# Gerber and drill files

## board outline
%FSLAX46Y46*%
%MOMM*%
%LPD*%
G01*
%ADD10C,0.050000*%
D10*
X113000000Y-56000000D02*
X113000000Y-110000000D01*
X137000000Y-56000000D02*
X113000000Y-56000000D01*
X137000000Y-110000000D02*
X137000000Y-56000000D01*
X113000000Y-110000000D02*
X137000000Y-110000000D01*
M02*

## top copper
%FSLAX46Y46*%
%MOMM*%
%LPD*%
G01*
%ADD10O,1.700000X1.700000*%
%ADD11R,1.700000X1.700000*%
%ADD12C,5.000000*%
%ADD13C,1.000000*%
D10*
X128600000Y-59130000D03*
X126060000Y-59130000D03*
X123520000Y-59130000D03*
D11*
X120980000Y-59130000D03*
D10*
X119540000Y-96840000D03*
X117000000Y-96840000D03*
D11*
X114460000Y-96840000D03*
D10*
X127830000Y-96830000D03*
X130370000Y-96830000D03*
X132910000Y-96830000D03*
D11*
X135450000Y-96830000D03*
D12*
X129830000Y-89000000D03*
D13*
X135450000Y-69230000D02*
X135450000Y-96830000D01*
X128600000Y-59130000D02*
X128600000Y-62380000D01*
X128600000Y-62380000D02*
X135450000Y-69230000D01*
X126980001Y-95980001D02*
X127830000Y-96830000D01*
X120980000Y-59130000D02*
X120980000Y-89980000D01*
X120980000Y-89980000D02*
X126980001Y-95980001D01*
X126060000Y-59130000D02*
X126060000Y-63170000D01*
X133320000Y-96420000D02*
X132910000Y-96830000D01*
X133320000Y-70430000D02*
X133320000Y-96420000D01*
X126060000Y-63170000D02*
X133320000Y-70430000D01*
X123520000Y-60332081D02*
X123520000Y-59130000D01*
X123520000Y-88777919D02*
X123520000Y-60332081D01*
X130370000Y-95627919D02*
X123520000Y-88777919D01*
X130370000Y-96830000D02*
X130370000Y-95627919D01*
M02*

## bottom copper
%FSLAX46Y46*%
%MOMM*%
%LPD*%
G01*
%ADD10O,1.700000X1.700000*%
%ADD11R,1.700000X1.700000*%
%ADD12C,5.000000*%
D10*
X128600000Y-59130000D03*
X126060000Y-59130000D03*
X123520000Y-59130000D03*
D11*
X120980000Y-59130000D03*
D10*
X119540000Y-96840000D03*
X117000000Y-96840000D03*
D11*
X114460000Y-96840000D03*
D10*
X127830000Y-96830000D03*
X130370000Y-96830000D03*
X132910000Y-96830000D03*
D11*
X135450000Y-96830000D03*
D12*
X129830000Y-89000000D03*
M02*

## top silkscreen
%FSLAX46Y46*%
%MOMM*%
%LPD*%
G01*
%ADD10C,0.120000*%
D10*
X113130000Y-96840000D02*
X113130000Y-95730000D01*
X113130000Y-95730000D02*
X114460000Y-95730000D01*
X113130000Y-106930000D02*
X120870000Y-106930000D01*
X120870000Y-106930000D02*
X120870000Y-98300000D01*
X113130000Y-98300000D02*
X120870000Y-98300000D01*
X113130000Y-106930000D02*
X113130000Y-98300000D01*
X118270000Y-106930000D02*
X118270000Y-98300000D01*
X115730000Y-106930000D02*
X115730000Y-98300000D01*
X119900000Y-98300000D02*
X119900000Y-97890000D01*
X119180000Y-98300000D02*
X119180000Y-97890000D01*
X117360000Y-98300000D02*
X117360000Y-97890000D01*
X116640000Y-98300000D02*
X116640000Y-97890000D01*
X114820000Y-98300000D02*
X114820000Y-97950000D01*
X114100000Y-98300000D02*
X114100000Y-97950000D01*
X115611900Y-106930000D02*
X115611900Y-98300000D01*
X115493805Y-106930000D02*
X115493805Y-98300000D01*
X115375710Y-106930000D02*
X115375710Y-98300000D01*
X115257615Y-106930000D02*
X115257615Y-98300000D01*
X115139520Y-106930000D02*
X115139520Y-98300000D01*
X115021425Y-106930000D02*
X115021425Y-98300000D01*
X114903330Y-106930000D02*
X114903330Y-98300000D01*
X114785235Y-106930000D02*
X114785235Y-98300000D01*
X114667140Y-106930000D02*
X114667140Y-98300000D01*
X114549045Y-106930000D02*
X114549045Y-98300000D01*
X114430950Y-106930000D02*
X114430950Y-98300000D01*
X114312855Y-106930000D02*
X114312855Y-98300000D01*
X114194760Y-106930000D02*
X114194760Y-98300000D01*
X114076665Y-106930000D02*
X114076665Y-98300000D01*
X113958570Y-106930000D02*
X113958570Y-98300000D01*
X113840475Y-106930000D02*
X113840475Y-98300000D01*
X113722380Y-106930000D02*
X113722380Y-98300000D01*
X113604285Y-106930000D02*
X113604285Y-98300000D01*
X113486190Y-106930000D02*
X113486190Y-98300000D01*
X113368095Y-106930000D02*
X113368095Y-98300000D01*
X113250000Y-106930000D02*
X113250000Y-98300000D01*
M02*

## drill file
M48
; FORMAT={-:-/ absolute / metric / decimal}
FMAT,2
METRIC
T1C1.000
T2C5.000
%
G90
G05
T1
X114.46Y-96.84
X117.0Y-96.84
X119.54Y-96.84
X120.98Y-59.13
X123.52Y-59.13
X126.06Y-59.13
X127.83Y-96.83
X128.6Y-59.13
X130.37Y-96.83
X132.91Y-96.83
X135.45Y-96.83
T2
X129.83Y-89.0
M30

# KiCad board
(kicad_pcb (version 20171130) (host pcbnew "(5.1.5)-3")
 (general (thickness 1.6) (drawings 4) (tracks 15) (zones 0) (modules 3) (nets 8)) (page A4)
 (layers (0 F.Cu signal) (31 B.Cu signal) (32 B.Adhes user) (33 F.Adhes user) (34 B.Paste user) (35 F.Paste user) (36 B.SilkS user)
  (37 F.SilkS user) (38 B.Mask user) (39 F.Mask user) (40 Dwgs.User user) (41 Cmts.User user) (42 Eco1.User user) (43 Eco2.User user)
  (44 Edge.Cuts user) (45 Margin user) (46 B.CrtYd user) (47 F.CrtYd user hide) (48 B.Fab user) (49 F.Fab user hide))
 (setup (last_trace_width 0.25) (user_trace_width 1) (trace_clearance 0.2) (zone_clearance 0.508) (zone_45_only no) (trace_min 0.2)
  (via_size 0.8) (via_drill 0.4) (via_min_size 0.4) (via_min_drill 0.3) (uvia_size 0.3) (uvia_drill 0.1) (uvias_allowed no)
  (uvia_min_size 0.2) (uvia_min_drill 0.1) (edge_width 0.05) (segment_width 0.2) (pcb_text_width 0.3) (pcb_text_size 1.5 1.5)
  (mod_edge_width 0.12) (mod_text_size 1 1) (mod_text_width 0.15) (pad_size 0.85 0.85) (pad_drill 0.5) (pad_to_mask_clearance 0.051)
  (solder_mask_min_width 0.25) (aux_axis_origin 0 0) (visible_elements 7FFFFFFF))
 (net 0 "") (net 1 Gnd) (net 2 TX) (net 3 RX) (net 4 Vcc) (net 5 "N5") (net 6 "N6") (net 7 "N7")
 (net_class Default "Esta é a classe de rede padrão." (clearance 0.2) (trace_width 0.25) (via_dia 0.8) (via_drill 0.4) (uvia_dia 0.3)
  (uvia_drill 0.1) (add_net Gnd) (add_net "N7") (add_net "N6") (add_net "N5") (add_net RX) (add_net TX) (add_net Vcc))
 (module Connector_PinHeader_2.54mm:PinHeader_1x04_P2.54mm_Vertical (layer B.Cu) (at 120.98 59.13 270)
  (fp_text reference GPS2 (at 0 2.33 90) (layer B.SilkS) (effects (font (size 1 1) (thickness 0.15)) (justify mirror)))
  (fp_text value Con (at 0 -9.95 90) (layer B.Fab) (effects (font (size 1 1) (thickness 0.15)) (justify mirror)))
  (pad 4 thru_hole oval (at 0 -7.62 270) (size 1.7 1.7) (drill 1) (layers *.Cu *.Mask) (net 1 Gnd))
  (pad 3 thru_hole oval (at 0 -5.08 270) (size 1.7 1.7) (drill 1) (layers *.Cu *.Mask) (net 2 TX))
  (pad 2 thru_hole oval (at 0 -2.54 270) (size 1.7 1.7) (drill 1) (layers *.Cu *.Mask) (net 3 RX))
  (pad 1 thru_hole rect (at 0 0 270) (size 1.7 1.7) (drill 1) (layers *.Cu *.Mask) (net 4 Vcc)))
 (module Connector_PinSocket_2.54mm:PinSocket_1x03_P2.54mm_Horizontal (layer F.Cu) (at 114.46 96.84 90)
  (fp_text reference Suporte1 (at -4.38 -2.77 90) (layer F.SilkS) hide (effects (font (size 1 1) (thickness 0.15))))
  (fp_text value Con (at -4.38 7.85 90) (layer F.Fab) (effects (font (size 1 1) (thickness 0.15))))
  (fp_line (start 0 -1.33) (end 1.11 -1.33) (layer F.SilkS) (width 0.12))
  (fp_line (start 1.11 -1.33) (end 1.11 0) (layer F.SilkS) (width 0.12))
  (fp_line (start -10.09 -1.33) (end -10.09 6.41) (layer F.SilkS) (width 0.12))
  (fp_line (start -10.09 6.41) (end -1.46 6.41) (layer F.SilkS) (width 0.12))
  (fp_line (start -1.46 -1.33) (end -1.46 6.41) (layer F.SilkS) (width 0.12))
  (fp_line (start -10.09 -1.33) (end -1.46 -1.33) (layer F.SilkS) (width 0.12))
  (fp_line (start -10.09 3.81) (end -1.46 3.81) (layer F.SilkS) (width 0.12))
  (fp_line (start -10.09 1.27) (end -1.46 1.27) (layer F.SilkS) (width 0.12))
  (fp_line (start -1.46 5.44) (end -1.05 5.44) (layer F.SilkS) (width 0.12))
  (fp_line (start -1.46 4.72) (end -1.05 4.72) (layer F.SilkS) (width 0.12))
  (fp_line (start -1.46 2.9) (end -1.05 2.9) (layer F.SilkS) (width 0.12))
  (fp_line (start -1.46 2.18) (end -1.05 2.18) (layer F.SilkS) (width 0.12))
  (fp_line (start -1.46 0.36) (end -1.11 0.36) (layer F.SilkS) (width 0.12))
  (fp_line (start -1.46 -0.36) (end -1.11 -0.36) (layer F.SilkS) (width 0.12))
  (fp_line (start -10.09 1.1519) (end -1.46 1.1519) (layer F.SilkS) (width 0.12))
  (fp_line (start -10.09 1.033805) (end -1.46 1.033805) (layer F.SilkS) (width 0.12))
  (fp_line (start -10.09 0.91571) (end -1.46 0.91571) (layer F.SilkS) (width 0.12))
  (fp_line (start -10.09 0.797615) (end -1.46 0.797615) (layer F.SilkS) (width 0.12))
  (fp_line (start -10.09 0.67952) (end -1.46 0.67952) (layer F.SilkS) (width 0.12))
  (fp_line (start -10.09 0.561425) (end -1.46 0.561425) (layer F.SilkS) (width 0.12))
  (fp_line (start -10.09 0.44333) (end -1.46 0.44333) (layer F.SilkS) (width 0.12))
  (fp_line (start -10.09 0.325235) (end -1.46 0.325235) (layer F.SilkS) (width 0.12))
  (fp_line (start -10.09 0.20714) (end -1.46 0.20714) (layer F.SilkS) (width 0.12))
  (fp_line (start -10.09 0.089045) (end -1.46 0.089045) (layer F.SilkS) (width 0.12))
  (fp_line (start -10.09 -0.02905) (end -1.46 -0.02905) (layer F.SilkS) (width 0.12))
  (fp_line (start -10.09 -0.147145) (end -1.46 -0.147145) (layer F.SilkS) (width 0.12))
  (fp_line (start -10.09 -0.26524) (end -1.46 -0.26524) (layer F.SilkS) (width 0.12))
  (fp_line (start -10.09 -0.383335) (end -1.46 -0.383335) (layer F.SilkS) (width 0.12))
  (fp_line (start -10.09 -0.50143) (end -1.46 -0.50143) (layer F.SilkS) (width 0.12))
  (fp_line (start -10.09 -0.619525) (end -1.46 -0.619525) (layer F.SilkS) (width 0.12))
  (fp_line (start -10.09 -0.73762) (end -1.46 -0.73762) (layer F.SilkS) (width 0.12))
  (fp_line (start -10.09 -0.855715) (end -1.46 -0.855715) (layer F.SilkS) (width 0.12))
  (fp_line (start -10.09 -0.97381) (end -1.46 -0.97381) (layer F.SilkS) (width 0.12))
  (fp_line (start -10.09 -1.091905) (end -1.46 -1.091905) (layer F.SilkS) (width 0.12))
  (fp_line (start -10.09 -1.21) (end -1.46 -1.21) (layer F.SilkS) (width 0.12))
  (pad 3 thru_hole oval (at 0 5.08 90) (size 1.7 1.7) (drill 1) (layers *.Cu *.Mask) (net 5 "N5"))
  (pad 2 thru_hole oval (at 0 2.54 90) (size 1.7 1.7) (drill 1) (layers *.Cu *.Mask) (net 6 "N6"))
  (pad 1 thru_hole rect (at 0 0 90) (size 1.7 1.7) (drill 1) (layers *.Cu *.Mask) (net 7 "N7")))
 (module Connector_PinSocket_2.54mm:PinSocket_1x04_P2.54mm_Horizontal (layer B.Cu) (at 135.45 96.83 90)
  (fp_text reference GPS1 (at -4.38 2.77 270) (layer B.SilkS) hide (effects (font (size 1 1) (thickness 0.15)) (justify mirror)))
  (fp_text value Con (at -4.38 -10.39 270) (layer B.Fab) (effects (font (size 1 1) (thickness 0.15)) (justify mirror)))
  (pad 4 thru_hole oval (at 0 -7.62 90) (size 1.7 1.7) (drill 1) (layers *.Cu *.Mask) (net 4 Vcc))
  (pad 3 thru_hole oval (at 0 -5.08 90) (size 1.7 1.7) (drill 1) (layers *.Cu *.Mask) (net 3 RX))
  (pad 2 thru_hole oval (at 0 -2.54 90) (size 1.7 1.7) (drill 1) (layers *.Cu *.Mask) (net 2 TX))
  (pad 1 thru_hole rect (at 0 0 90) (size 1.7 1.7) (drill 1) (layers *.Cu *.Mask) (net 1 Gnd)))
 (gr_line (start 113 56) (end 113 110) (layer Edge.Cuts) (width 0.05))
 (gr_line (start 137 56) (end 113 56) (layer Edge.Cuts) (width 0.05))
 (gr_line (start 137 110) (end 137 56) (layer Edge.Cuts) (width 0.05))
 (gr_line (start 113 110) (end 137 110) (layer Edge.Cuts) (width 0.05))
 (via (at 129.83 89) (size 5) (drill 4.9999) (layers F.Cu B.Cu) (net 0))
 (segment (start 135.45 69.23) (end 135.45 96.83) (width 1) (layer F.Cu) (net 1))
 (segment (start 128.6 59.13) (end 128.6 62.38) (width 1) (layer F.Cu) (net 1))
 (segment (start 128.6 62.38) (end 135.45 69.23) (width 1) (layer F.Cu) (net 1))
 (segment (start 126.980001 95.980001) (end 127.83 96.83) (width 1) (layer F.Cu) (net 4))
 (segment (start 120.98 59.13) (end 120.98 89.98) (width 1) (layer F.Cu) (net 4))
 (segment (start 120.98 89.98) (end 126.980001 95.980001) (width 1) (layer F.Cu) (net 4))
 (segment (start 126.06 59.13) (end 126.06 63.17) (width 1) (layer F.Cu) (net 2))
 (segment (start 133.32 96.42) (end 132.91 96.83) (width 1) (layer F.Cu) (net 2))
 (segment (start 133.32 70.43) (end 133.32 96.42) (width 1) (layer F.Cu) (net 2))
 (segment (start 126.06 63.17) (end 133.32 70.43) (width 1) (layer F.Cu) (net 2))
 (segment (start 123.52 60.332081) (end 123.52 59.13) (width 1) (layer F.Cu) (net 3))
 (segment (start 123.52 88.777919) (end 123.52 60.332081) (width 1) (layer F.Cu) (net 3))
 (segment (start 130.37 95.627919) (end 123.52 88.777919) (width 1) (layer F.Cu) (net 3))
 (segment (start 130.37 96.83) (end 130.37 95.627919) (width 1) (layer F.Cu) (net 3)))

